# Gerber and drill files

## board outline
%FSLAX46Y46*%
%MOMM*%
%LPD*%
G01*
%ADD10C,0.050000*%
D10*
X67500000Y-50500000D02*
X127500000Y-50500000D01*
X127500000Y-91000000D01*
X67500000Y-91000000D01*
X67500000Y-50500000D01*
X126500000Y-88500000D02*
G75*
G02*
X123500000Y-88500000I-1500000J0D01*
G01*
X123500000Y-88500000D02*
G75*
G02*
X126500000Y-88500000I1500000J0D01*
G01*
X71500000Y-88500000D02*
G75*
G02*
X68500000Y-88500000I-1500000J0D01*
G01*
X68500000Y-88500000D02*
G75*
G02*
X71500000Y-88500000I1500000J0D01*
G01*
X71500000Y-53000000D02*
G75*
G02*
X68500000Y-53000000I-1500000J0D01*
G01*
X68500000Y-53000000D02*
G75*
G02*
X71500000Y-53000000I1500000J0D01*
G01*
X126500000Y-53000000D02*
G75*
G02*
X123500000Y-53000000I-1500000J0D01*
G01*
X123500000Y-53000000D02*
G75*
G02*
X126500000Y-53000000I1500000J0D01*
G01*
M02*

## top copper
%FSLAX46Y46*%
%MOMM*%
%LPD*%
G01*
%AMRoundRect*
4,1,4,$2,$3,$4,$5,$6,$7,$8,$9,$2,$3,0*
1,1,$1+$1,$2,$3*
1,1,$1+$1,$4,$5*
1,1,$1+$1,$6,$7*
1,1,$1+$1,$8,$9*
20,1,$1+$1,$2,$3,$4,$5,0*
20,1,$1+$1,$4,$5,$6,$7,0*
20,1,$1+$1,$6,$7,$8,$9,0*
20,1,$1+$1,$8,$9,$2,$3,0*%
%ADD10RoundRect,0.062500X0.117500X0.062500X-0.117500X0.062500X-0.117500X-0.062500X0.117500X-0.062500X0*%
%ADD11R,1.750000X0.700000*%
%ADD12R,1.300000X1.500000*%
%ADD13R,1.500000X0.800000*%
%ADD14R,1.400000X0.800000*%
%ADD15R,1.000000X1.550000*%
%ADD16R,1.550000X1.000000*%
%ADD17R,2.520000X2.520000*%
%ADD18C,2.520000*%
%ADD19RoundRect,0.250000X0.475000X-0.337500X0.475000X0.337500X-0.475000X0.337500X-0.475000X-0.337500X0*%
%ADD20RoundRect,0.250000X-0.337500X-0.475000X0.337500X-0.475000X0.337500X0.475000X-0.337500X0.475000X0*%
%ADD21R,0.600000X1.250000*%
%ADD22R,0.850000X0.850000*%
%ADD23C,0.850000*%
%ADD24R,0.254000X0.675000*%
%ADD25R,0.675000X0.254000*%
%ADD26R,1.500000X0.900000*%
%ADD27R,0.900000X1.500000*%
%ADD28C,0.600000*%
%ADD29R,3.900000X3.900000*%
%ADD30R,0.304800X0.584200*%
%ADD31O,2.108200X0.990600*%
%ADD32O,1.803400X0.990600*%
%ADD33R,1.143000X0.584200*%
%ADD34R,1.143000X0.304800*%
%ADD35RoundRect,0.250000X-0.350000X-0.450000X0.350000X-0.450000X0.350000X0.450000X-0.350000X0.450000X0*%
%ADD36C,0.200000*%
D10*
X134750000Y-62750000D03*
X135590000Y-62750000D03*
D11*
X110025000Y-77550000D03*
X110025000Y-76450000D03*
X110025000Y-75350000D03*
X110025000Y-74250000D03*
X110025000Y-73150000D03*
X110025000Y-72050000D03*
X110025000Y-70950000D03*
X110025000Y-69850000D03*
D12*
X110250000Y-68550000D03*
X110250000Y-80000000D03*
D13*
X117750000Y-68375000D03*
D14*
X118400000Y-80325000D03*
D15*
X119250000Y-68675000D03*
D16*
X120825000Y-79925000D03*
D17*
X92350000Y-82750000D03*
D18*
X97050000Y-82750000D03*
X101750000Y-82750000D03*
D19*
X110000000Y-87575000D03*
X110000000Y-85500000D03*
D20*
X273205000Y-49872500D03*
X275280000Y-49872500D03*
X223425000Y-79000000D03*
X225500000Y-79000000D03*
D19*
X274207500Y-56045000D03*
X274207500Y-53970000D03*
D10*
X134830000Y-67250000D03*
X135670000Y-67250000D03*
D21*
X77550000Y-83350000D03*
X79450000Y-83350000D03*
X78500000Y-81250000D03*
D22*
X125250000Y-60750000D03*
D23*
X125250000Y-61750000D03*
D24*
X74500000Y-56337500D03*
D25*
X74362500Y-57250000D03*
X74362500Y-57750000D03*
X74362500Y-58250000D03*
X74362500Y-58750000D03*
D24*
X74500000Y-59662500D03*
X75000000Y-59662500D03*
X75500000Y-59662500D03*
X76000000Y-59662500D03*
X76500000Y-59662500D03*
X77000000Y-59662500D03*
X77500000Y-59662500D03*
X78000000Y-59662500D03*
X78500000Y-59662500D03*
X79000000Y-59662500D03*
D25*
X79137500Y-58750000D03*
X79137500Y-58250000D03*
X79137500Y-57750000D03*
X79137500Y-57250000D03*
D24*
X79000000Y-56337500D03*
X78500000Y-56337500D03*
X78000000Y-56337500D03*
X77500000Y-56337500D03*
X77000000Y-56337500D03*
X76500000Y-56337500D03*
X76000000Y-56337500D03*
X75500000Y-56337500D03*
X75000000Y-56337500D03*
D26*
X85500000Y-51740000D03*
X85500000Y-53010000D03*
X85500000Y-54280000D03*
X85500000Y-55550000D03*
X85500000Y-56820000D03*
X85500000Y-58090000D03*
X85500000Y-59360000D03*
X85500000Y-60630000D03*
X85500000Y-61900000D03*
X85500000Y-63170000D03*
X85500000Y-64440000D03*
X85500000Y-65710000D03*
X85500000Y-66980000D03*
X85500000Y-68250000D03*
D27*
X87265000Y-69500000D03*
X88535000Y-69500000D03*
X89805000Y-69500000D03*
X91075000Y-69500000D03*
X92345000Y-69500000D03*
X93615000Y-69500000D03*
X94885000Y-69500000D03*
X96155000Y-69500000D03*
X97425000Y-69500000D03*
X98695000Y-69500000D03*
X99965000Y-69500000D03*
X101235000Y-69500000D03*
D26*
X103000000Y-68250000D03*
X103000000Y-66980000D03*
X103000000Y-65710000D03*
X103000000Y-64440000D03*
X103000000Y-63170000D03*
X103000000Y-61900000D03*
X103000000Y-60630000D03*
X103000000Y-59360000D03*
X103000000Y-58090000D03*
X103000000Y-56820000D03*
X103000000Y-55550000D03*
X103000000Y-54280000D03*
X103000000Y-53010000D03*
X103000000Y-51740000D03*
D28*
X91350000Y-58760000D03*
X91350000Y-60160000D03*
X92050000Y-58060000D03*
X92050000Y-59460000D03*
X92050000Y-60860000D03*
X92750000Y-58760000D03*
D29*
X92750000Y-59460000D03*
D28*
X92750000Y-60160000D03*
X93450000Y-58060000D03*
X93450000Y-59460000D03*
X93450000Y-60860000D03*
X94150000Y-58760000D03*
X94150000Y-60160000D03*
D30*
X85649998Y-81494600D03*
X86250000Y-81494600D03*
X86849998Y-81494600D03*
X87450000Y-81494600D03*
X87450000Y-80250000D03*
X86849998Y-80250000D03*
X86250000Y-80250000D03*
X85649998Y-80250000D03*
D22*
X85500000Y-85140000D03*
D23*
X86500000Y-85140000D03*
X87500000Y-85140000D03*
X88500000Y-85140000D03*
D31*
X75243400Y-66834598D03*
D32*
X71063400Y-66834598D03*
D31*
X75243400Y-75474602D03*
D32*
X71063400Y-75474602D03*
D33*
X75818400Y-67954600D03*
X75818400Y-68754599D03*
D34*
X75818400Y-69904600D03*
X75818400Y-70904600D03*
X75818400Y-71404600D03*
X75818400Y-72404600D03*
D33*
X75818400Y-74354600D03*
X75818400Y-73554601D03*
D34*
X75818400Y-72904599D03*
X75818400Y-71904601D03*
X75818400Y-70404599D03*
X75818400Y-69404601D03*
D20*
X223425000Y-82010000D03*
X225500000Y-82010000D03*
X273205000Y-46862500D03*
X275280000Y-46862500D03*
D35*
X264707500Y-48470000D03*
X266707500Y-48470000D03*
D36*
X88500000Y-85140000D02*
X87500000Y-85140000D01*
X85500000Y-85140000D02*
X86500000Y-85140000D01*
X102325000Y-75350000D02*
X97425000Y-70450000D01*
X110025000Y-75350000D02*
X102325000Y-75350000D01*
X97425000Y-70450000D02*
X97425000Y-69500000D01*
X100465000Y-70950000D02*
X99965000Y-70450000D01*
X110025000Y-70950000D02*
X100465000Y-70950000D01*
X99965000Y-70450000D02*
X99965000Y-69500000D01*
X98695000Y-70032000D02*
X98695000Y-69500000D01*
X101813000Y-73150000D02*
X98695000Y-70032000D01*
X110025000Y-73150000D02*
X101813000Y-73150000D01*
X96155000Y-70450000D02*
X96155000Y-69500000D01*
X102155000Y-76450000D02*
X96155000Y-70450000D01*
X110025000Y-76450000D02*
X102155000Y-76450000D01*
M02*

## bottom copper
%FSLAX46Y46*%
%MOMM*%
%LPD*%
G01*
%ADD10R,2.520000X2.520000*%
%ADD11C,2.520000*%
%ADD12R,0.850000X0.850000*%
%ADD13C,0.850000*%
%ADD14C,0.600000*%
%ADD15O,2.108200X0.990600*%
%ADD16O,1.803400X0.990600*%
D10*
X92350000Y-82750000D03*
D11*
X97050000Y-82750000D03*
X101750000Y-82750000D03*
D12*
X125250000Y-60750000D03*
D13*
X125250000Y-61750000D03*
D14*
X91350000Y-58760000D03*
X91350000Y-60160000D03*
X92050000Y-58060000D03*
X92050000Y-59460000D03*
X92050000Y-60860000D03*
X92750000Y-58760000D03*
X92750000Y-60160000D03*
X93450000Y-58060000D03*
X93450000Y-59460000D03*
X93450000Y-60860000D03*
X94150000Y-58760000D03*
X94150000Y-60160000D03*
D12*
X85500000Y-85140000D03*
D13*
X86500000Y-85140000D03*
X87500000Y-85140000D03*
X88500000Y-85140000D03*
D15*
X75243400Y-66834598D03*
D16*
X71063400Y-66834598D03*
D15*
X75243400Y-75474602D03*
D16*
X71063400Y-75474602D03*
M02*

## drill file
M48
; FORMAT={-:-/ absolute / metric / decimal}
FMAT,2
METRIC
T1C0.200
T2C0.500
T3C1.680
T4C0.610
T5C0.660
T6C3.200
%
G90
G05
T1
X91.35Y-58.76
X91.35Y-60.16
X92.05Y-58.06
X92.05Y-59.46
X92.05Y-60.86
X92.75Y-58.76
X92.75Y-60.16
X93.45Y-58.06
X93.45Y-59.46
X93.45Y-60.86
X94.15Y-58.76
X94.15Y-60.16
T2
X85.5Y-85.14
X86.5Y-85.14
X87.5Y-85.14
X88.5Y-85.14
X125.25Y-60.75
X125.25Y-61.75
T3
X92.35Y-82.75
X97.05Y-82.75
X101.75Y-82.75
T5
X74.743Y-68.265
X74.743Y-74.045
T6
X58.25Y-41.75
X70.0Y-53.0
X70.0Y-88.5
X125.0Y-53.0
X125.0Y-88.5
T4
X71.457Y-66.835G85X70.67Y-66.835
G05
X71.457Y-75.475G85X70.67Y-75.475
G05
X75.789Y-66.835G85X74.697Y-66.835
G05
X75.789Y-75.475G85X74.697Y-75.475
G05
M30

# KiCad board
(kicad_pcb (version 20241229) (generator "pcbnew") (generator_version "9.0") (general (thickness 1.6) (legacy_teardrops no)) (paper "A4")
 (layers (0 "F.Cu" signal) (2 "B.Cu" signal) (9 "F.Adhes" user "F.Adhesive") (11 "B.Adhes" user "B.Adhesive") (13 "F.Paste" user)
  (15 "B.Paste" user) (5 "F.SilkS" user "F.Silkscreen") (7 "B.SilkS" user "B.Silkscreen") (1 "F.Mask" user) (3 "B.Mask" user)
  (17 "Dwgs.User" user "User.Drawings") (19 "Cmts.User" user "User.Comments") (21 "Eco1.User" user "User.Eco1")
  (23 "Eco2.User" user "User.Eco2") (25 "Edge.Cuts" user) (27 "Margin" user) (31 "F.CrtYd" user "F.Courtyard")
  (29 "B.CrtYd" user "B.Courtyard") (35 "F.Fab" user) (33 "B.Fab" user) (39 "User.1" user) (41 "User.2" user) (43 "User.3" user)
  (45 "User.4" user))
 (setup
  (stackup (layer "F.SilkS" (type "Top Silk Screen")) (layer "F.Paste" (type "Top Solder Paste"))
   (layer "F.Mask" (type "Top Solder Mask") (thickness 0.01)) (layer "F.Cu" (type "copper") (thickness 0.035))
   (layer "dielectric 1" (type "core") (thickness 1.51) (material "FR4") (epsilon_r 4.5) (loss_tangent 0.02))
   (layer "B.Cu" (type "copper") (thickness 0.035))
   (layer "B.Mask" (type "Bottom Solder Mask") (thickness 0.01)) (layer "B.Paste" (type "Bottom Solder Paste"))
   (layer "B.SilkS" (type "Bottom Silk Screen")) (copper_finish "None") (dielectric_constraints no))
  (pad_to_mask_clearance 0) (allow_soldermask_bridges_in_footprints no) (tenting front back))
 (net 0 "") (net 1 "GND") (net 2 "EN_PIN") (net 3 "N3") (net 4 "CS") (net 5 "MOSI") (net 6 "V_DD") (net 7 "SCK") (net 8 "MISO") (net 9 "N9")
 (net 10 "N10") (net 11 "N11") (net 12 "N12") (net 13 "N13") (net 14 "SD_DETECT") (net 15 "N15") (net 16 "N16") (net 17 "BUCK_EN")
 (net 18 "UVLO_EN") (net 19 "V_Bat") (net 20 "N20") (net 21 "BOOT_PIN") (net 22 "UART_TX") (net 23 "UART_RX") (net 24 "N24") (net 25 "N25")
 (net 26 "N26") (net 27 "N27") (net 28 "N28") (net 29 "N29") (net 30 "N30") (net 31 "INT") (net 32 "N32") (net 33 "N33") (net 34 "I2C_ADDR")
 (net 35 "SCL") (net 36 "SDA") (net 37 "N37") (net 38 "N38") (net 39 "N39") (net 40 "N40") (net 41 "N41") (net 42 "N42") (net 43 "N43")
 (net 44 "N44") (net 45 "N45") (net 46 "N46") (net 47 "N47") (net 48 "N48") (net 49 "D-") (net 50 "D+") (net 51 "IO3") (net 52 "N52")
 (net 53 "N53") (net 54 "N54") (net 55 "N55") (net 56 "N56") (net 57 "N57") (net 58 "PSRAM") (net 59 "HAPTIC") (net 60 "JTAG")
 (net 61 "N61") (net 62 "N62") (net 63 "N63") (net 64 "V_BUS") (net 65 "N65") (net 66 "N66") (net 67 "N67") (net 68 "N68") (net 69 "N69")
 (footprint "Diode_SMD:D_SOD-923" (layer "F.Cu") (at 135.17 62.75)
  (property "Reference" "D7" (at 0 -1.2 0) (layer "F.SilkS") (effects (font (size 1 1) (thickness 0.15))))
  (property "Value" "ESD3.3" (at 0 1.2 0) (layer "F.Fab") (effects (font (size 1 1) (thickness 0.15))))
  (pad "1" smd roundrect (at -0.42 0 180) (size 0.36 0.25) (layers "F.Cu" "F.Mask" "F.Paste") (roundrect_rratio 0.25) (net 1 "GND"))
  (pad "2" smd roundrect (at 0.42 0 180) (size 0.36 0.25) (layers "F.Cu" "F.Mask" "F.Paste") (roundrect_rratio 0.25) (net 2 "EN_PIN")))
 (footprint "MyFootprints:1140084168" (layer "F.Cu") (at 115.375 74.275 -90)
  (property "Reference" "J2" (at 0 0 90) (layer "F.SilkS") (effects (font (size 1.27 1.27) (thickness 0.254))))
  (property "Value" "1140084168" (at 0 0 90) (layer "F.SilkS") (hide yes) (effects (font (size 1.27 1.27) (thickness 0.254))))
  (pad "1" smd rect (at 3.275 5.35 270) (size 0.7 1.75) (layers "F.Cu" "F.Mask" "F.Paste") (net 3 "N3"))
  (pad "2" smd rect (at 2.175 5.35 270) (size 0.7 1.75) (layers "F.Cu" "F.Mask" "F.Paste") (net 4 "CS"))
  (pad "3" smd rect (at 1.075 5.35 270) (size 0.7 1.75) (layers "F.Cu" "F.Mask" "F.Paste") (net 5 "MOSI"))
  (pad "4" smd rect (at -0.025 5.35 270) (size 0.7 1.75) (layers "F.Cu" "F.Mask" "F.Paste") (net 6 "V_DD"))
  (pad "5" smd rect (at -1.125 5.35 270) (size 0.7 1.75) (layers "F.Cu" "F.Mask" "F.Paste") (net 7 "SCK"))
  (pad "6" smd rect (at -2.225 5.35 270) (size 0.7 1.75) (layers "F.Cu" "F.Mask" "F.Paste") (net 1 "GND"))
  (pad "7" smd rect (at -3.325 5.35 270) (size 0.7 1.75) (layers "F.Cu" "F.Mask" "F.Paste") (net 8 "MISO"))
  (pad "8" smd rect (at -4.425 5.35 270) (size 0.7 1.75) (layers "F.Cu" "F.Mask" "F.Paste") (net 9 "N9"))
  (pad "9" smd rect (at -5.725 5.125) (size 1.3 1.5) (layers "F.Cu" "F.Mask" "F.Paste") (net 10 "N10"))
  (pad "10" smd rect (at 5.725 5.125) (size 1.3 1.5) (layers "F.Cu" "F.Mask" "F.Paste") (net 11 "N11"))
  (pad "11" smd rect (at -5.9 -2.375 270) (size 0.8 1.5) (layers "F.Cu" "F.Mask" "F.Paste") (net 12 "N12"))
  (pad "12" smd rect (at 6.05 -3.025 270) (size 0.8 1.4) (layers "F.Cu" "F.Mask" "F.Paste") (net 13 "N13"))
  (pad "CD1" smd rect (at -5.6 -3.875) (size 1 1.55) (layers "F.Cu" "F.Mask" "F.Paste") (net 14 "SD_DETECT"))
  (pad "CD2" smd rect (at 5.65 -5.45 270) (size 1 1.55) (layers "F.Cu" "F.Mask" "F.Paste") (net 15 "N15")))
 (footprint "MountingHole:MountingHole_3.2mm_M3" (layer "F.Cu") (at 58.25 41.75)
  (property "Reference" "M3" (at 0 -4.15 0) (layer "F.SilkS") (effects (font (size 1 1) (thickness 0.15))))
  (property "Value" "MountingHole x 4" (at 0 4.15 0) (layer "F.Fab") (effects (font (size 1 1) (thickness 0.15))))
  (pad "" np_thru_hole circle (at 0 0) (size 3.2 3.2) (drill 3.2) (layers "*.Cu" "*.Mask")))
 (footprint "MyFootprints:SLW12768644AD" (layer "F.Cu") (at 92.35 82.75)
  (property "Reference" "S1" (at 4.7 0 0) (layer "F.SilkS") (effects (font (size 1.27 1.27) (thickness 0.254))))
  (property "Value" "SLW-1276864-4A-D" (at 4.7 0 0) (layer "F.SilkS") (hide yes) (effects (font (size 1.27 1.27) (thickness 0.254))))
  (pad "1" thru_hole rect (at 0 0) (size 2.52 2.52) (drill 1.68) (layers "*.Cu" "*.Mask") (remove_unused_layers no) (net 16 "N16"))
  (pad "2" thru_hole circle (at 4.7 0) (size 2.52 2.52) (drill 1.68) (layers "*.Cu" "*.Mask") (remove_unused_layers no) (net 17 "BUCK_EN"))
  (pad "3" thru_hole circle (at 9.4 0) (size 2.52 2.52) (drill 1.68) (layers "*.Cu" "*.Mask") (remove_unused_layers no) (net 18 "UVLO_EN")))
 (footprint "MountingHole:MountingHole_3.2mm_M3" (layer "F.Cu") (at 70 88.5)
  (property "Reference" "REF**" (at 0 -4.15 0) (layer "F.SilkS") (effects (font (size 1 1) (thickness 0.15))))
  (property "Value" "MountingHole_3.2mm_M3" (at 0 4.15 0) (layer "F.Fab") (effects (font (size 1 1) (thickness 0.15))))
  (pad "" np_thru_hole circle (at 0 0) (size 3.2 3.2) (drill 3.2) (layers "*.Cu" "*.Mask")))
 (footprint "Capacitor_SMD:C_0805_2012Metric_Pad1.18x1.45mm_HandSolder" (layer "F.Cu") (at 110 86.5375 90)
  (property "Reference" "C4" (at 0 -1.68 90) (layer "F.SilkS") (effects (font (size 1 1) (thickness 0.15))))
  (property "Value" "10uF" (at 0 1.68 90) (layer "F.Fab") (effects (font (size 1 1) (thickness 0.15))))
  (pad "1" smd roundrect (at -1.0375 0 90) (size 1.175 1.45) (layers "F.Cu" "F.Mask" "F.Paste") (roundrect_rratio 0.212766) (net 6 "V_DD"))
  (pad "2" smd roundrect (at 1.0375 0 90) (size 1.175 1.45) (layers "F.Cu" "F.Mask" "F.Paste") (roundrect_rratio 0.212766) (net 1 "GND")))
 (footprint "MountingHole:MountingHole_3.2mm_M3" (layer "F.Cu") (at 125 88.5)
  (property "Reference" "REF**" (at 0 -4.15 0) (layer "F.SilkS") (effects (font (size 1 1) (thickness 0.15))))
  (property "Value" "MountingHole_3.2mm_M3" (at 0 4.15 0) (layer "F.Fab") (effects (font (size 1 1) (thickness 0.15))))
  (pad "" np_thru_hole circle (at 0 0) (size 3.2 3.2) (drill 3.2) (layers "*.Cu" "*.Mask")))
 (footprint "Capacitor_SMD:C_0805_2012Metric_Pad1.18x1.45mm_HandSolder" (layer "F.Cu") (at 274.2425 49.8725)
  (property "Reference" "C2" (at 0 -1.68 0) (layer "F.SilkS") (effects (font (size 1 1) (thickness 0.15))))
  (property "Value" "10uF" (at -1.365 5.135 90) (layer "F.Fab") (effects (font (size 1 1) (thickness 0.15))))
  (pad "1" smd roundrect (at -1.0375 0) (size 1.175 1.45) (layers "F.Cu" "F.Mask" "F.Paste") (roundrect_rratio 0.212766) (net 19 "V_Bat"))
  (pad "2" smd roundrect (at 1.0375 0) (size 1.175 1.45) (layers "F.Cu" "F.Mask" "F.Paste") (roundrect_rratio 0.212766) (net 1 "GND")))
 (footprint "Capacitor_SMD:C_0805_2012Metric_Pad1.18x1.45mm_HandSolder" (layer "F.Cu") (at 224.4625 79)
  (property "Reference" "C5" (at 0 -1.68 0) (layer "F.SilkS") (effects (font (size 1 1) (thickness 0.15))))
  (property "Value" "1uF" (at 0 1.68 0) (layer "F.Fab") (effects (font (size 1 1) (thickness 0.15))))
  (pad "1" smd roundrect (at -1.0375 0) (size 1.175 1.45) (layers "F.Cu" "F.Mask" "F.Paste") (roundrect_rratio 0.212766) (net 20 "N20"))
  (pad "2" smd roundrect (at 1.0375 0) (size 1.175 1.45) (layers "F.Cu" "F.Mask" "F.Paste") (roundrect_rratio 0.212766) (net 1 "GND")))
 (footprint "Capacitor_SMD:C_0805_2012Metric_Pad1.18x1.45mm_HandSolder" (layer "F.Cu") (at 274.2075 55.0075 90)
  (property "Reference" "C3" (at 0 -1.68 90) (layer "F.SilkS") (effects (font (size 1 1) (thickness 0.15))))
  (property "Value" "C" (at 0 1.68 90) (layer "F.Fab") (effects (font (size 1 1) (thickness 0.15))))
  (pad "1" smd roundrect (at -1.0375 0 90) (size 1.175 1.45) (layers "F.Cu" "F.Mask" "F.Paste") (roundrect_rratio 0.212766) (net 6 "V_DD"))
  (pad "2" smd roundrect (at 1.0375 0 90) (size 1.175 1.45) (layers "F.Cu" "F.Mask" "F.Paste") (roundrect_rratio 0.212766) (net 1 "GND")))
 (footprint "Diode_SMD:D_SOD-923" (layer "F.Cu") (at 135.25 67.25)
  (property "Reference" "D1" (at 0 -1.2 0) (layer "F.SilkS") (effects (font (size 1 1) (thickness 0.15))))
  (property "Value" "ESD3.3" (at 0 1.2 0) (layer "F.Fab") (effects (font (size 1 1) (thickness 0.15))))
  (pad "1" smd roundrect (at -0.42 0 180) (size 0.36 0.25) (layers "F.Cu" "F.Mask" "F.Paste") (roundrect_rratio 0.25) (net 1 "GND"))
  (pad "2" smd roundrect (at 0.42 0 180) (size 0.36 0.25) (layers "F.Cu" "F.Mask" "F.Paste") (roundrect_rratio 0.25) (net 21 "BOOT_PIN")))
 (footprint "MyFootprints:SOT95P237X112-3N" (layer "F.Cu") (at 78.5 82.3 90)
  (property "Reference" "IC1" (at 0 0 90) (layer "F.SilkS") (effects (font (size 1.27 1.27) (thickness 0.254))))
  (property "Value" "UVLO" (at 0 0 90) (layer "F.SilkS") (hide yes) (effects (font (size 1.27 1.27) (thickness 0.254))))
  (pad "1" smd rect (at -1.05 -0.95 180) (size 0.6 1.25) (layers "F.Cu" "F.Mask" "F.Paste") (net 18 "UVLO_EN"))
  (pad "2" smd rect (at -1.05 0.95 180) (size 0.6 1.25) (layers "F.Cu" "F.Mask" "F.Paste") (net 19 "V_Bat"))
  (pad "3" smd rect (at 1.05 0 180) (size 0.6 1.25) (layers "F.Cu" "F.Mask" "F.Paste") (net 1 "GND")))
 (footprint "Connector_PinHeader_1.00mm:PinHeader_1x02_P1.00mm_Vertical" (layer "F.Cu") (at 125.25 60.75)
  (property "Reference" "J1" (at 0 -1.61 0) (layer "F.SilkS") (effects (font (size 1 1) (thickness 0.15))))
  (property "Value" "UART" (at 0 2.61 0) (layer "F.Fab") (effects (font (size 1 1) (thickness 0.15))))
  (pad "1" thru_hole rect (at 0 0) (size 0.85 0.85) (drill 0.5) (layers "*.Cu" "*.Mask") (remove_unused_layers no) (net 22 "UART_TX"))
  (pad "2" thru_hole circle (at 0 1) (size 0.85 0.85) (drill 0.5) (layers "*.Cu" "*.Mask") (remove_unused_layers no) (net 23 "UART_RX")))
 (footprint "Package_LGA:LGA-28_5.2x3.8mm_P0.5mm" (layer "F.Cu") (at 76.75 58)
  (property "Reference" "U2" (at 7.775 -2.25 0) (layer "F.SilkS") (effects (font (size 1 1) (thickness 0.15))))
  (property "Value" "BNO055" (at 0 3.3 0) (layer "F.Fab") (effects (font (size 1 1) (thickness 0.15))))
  (pad "1" smd rect (at -2.25 -1.6625) (size 0.254 0.675) (layers "F.Cu" "F.Mask" "F.Paste") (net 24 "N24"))
  (pad "2" smd rect (at -2.3875 -0.75 90) (size 0.254 0.675) (layers "F.Cu" "F.Mask" "F.Paste") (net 1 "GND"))
  (pad "3" smd rect (at -2.3875 -0.25 90) (size 0.254 0.675) (layers "F.Cu" "F.Mask" "F.Paste") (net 6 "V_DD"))
  (pad "4" smd rect (at -2.3875 0.25 90) (size 0.254 0.675) (layers "F.Cu" "F.Mask" "F.Paste") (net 6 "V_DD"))
  (pad "5" smd rect (at -2.3875 0.75 90) (size 0.254 0.675) (layers "F.Cu" "F.Mask" "F.Paste") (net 1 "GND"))
  (pad "6" smd rect (at -2.25 1.6625) (size 0.254 0.675) (layers "F.Cu" "F.Mask" "F.Paste") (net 1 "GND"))
  (pad "7" smd rect (at -1.75 1.6625) (size 0.254 0.675) (layers "F.Cu" "F.Mask" "F.Paste") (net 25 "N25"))
  (pad "8" smd rect (at -1.25 1.6625) (size 0.254 0.675) (layers "F.Cu" "F.Mask" "F.Paste") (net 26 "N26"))
  (pad "9" smd rect (at -0.75 1.6625) (size 0.254 0.675) (layers "F.Cu" "F.Mask" "F.Paste") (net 20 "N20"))
  (pad "10" smd rect (at -0.25 1.6625) (size 0.254 0.675) (layers "F.Cu" "F.Mask" "F.Paste") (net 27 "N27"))
  (pad "11" smd rect (at 0.25 1.6625) (size 0.254 0.675) (layers "F.Cu" "F.Mask" "F.Paste") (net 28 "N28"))
  (pad "12" smd rect (at 0.75 1.6625) (size 0.254 0.675) (layers "F.Cu" "F.Mask" "F.Paste") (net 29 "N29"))
  (pad "13" smd rect (at 1.25 1.6625) (size 0.254 0.675) (layers "F.Cu" "F.Mask" "F.Paste") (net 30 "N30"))
  (pad "14" smd rect (at 1.75 1.6625) (size 0.254 0.675) (layers "F.Cu" "F.Mask" "F.Paste") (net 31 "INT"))
  (pad "15" smd rect (at 2.25 1.6625) (size 0.254 0.675) (layers "F.Cu" "F.Mask" "F.Paste") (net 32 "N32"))
  (pad "16" smd rect (at 2.3875 0.75 90) (size 0.254 0.675) (layers "F.Cu" "F.Mask" "F.Paste") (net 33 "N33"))
  (pad "17" smd rect (at 2.3875 0.25 90) (size 0.254 0.675) (layers "F.Cu" "F.Mask" "F.Paste") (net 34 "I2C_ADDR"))
  (pad "18" smd rect (at 2.3875 -0.25 90) (size 0.254 0.675) (layers "F.Cu" "F.Mask" "F.Paste") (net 1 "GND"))
  (pad "19" smd rect (at 2.3875 -0.75 90) (size 0.254 0.675) (layers "F.Cu" "F.Mask" "F.Paste") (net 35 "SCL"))
  (pad "20" smd rect (at 2.25 -1.6625) (size 0.254 0.675) (layers "F.Cu" "F.Mask" "F.Paste") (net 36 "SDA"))
  (pad "21" smd rect (at 1.75 -1.6625) (size 0.254 0.675) (layers "F.Cu" "F.Mask" "F.Paste") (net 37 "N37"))
  (pad "22" smd rect (at 1.25 -1.6625) (size 0.254 0.675) (layers "F.Cu" "F.Mask" "F.Paste") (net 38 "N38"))
  (pad "23" smd rect (at 0.75 -1.6625) (size 0.254 0.675) (layers "F.Cu" "F.Mask" "F.Paste") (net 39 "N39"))
  (pad "24" smd rect (at 0.25 -1.6625) (size 0.254 0.675) (layers "F.Cu" "F.Mask" "F.Paste") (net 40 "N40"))
  (pad "25" smd rect (at -0.25 -1.6625) (size 0.254 0.675) (layers "F.Cu" "F.Mask" "F.Paste") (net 1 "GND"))
  (pad "26" smd rect (at -0.75 -1.6625) (size 0.254 0.675) (layers "F.Cu" "F.Mask" "F.Paste") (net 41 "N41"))
  (pad "27" smd rect (at -1.25 -1.6625) (size 0.254 0.675) (layers "F.Cu" "F.Mask" "F.Paste") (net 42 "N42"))
  (pad "28" smd rect (at -1.75 -1.6625) (size 0.254 0.675) (layers "F.Cu" "F.Mask" "F.Paste") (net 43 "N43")))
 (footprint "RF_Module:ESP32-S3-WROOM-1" (layer "F.Cu") (at 94.25 57)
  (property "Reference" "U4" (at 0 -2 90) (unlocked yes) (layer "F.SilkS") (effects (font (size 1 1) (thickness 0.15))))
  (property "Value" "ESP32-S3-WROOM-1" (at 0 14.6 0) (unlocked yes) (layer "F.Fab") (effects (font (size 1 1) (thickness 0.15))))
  (pad "" smd rect (at -2.9 1.06) (size 0.9 0.9) (layers "F.Paste"))
  (pad "" smd rect (at -2.9 2.46 270) (size 0.9 0.9) (layers "F.Paste"))
  (pad "" smd rect (at -2.9 3.86) (size 0.9 0.9) (layers "F.Paste"))
  (pad "" smd rect (at -1.5 1.06 270) (size 0.9 0.9) (layers "F.Paste"))
  (pad "" smd rect (at -1.5 2.46 270) (size 0.9 0.9) (layers "F.Paste"))
  (pad "" smd rect (at -1.5 3.86 270) (size 0.9 0.9) (layers "F.Paste"))
  (pad "" smd rect (at -0.1 1.06 270) (size 0.9 0.9) (layers "F.Paste"))
  (pad "" smd rect (at -0.1 2.46 270) (size 0.9 0.9) (layers "F.Paste"))
  (pad "" smd rect (at -0.1 3.86 270) (size 0.9 0.9) (layers "F.Paste"))
  (pad "1" smd rect (at -8.75 -5.26) (size 1.5 0.9) (layers "F.Cu" "F.Mask" "F.Paste") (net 1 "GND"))
  (pad "2" smd rect (at -8.75 -3.99) (size 1.5 0.9) (layers "F.Cu" "F.Mask" "F.Paste") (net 6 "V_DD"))
  (pad "3" smd rect (at -8.75 -2.72) (size 1.5 0.9) (layers "F.Cu" "F.Mask" "F.Paste") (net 2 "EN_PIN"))
  (pad "4" smd rect (at -8.75 -1.45) (size 1.5 0.9) (layers "F.Cu" "F.Mask" "F.Paste") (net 36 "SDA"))
  (pad "5" smd rect (at -8.75 -0.18) (size 1.5 0.9) (layers "F.Cu" "F.Mask" "F.Paste") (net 35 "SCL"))
  (pad "6" smd rect (at -8.75 1.09) (size 1.5 0.9) (layers "F.Cu" "F.Mask" "F.Paste") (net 34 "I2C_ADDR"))
  (pad "7" smd rect (at -8.75 2.36) (size 1.5 0.9) (layers "F.Cu" "F.Mask" "F.Paste") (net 31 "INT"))
  (pad "8" smd rect (at -8.75 3.63) (size 1.5 0.9) (layers "F.Cu" "F.Mask" "F.Paste") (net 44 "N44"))
  (pad "9" smd rect (at -8.75 4.9) (size 1.5 0.9) (layers "F.Cu" "F.Mask" "F.Paste") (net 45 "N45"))
  (pad "10" smd rect (at -8.75 6.17) (size 1.5 0.9) (layers "F.Cu" "F.Mask" "F.Paste") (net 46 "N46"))
  (pad "11" smd rect (at -8.75 7.44) (size 1.5 0.9) (layers "F.Cu" "F.Mask" "F.Paste") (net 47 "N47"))
  (pad "12" smd rect (at -8.75 8.71) (size 1.5 0.9) (layers "F.Cu" "F.Mask" "F.Paste") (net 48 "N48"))
  (pad "13" smd rect (at -8.75 9.98) (size 1.5 0.9) (layers "F.Cu" "F.Mask" "F.Paste") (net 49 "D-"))
  (pad "14" smd rect (at -8.75 11.25 180) (size 1.5 0.9) (layers "F.Cu" "F.Mask" "F.Paste") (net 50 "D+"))
  (pad "15" smd rect (at -6.985 12.5 270) (size 1.5 0.9) (layers "F.Cu" "F.Mask" "F.Paste") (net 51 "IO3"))
  (pad "16" smd rect (at -5.715 12.5 270) (size 1.5 0.9) (layers "F.Cu" "F.Mask" "F.Paste") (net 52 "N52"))
  (pad "17" smd rect (at -4.445 12.5 270) (size 1.5 0.9) (layers "F.Cu" "F.Mask" "F.Paste") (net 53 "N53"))
  (pad "18" smd rect (at -3.175 12.5 270) (size 1.5 0.9) (layers "F.Cu" "F.Mask" "F.Paste") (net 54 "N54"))
  (pad "19" smd rect (at -1.905 12.5 270) (size 1.5 0.9) (layers "F.Cu" "F.Mask" "F.Paste") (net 14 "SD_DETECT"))
  (pad "20" smd rect (at -0.635 12.5 270) (size 1.5 0.9) (layers "F.Cu" "F.Mask" "F.Paste") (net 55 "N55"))
  (pad "21" smd rect (at 0.635 12.5 270) (size 1.5 0.9) (layers "F.Cu" "F.Mask" "F.Paste") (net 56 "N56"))
  (pad "22" smd rect (at 1.905 12.5 270) (size 1.5 0.9) (layers "F.Cu" "F.Mask" "F.Paste") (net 4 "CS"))
  (pad "23" smd rect (at 3.175 12.5 270) (size 1.5 0.9) (layers "F.Cu" "F.Mask" "F.Paste") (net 5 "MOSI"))
  (pad "24" smd rect (at 4.445 12.5 270) (size 1.5 0.9) (layers "F.Cu" "F.Mask" "F.Paste") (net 7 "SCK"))
  (pad "25" smd rect (at 5.715 12.5 270) (size 1.5 0.9) (layers "F.Cu" "F.Mask" "F.Paste") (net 8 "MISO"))
  (pad "26" smd rect (at 6.985 12.5 270) (size 1.5 0.9) (layers "F.Cu" "F.Mask" "F.Paste") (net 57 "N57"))
  (pad "27" smd rect (at 8.75 11.25) (size 1.5 0.9) (layers "F.Cu" "F.Mask" "F.Paste") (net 21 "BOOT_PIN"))
  (pad "28" smd rect (at 8.75 9.98) (size 1.5 0.9) (layers "F.Cu" "F.Mask" "F.Paste") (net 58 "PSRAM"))
  (pad "29" smd rect (at 8.75 8.71) (size 1.5 0.9) (layers "F.Cu" "F.Mask" "F.Paste") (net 58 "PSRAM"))
  (pad "30" smd rect (at 8.75 7.44) (size 1.5 0.9) (layers "F.Cu" "F.Mask" "F.Paste") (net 58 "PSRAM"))
  (pad "31" smd rect (at 8.75 6.17) (size 1.5 0.9) (layers "F.Cu" "F.Mask" "F.Paste") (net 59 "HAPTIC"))
  (pad "32" smd rect (at 8.75 4.9) (size 1.5 0.9) (layers "F.Cu" "F.Mask" "F.Paste") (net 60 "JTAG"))
  (pad "33" smd rect (at 8.75 3.63) (size 1.5 0.9) (layers "F.Cu" "F.Mask" "F.Paste") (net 60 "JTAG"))
  (pad "34" smd rect (at 8.75 2.36) (size 1.5 0.9) (layers "F.Cu" "F.Mask" "F.Paste") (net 60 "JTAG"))
  (pad "35" smd rect (at 8.75 1.09) (size 1.5 0.9) (layers "F.Cu" "F.Mask" "F.Paste") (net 60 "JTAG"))
  (pad "36" smd rect (at 8.75 -0.18) (size 1.5 0.9) (layers "F.Cu" "F.Mask" "F.Paste") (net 23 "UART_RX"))
  (pad "37" smd rect (at 8.75 -1.45) (size 1.5 0.9) (layers "F.Cu" "F.Mask" "F.Paste") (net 22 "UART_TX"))
  (pad "38" smd rect (at 8.75 -2.72) (size 1.5 0.9) (layers "F.Cu" "F.Mask" "F.Paste") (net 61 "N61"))
  (pad "39" smd rect (at 8.75 -3.99) (size 1.5 0.9) (layers "F.Cu" "F.Mask" "F.Paste") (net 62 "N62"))
  (pad "40" smd rect (at 8.75 -5.26) (size 1.5 0.9) (layers "F.Cu" "F.Mask" "F.Paste") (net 1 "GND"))
  (pad "41" thru_hole circle (at -2.9 1.76 90) (size 0.6 0.6) (drill 0.2) (layers "*.Cu" "F.Mask") (remove_unused_layers no) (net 1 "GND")
   (zone_connect 2))
  (pad "41" thru_hole circle (at -2.9 3.16) (size 0.6 0.6) (drill 0.2) (layers "*.Cu" "F.Mask") (remove_unused_layers no) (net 1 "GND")
   (zone_connect 2))
  (pad "41" thru_hole circle (at -2.2 1.06) (size 0.6 0.6) (drill 0.2) (layers "*.Cu" "F.Mask") (remove_unused_layers no) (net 1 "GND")
   (zone_connect 2))
  (pad "41" thru_hole circle (at -2.2 2.46) (size 0.6 0.6) (drill 0.2) (layers "*.Cu" "F.Mask") (remove_unused_layers no) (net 1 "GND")
   (zone_connect 2))
  (pad "41" thru_hole circle (at -2.2 3.86) (size 0.6 0.6) (drill 0.2) (layers "*.Cu" "F.Mask") (remove_unused_layers no) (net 1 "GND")
   (zone_connect 2))
  (pad "41" thru_hole circle (at -1.5 1.76) (size 0.6 0.6) (drill 0.2) (layers "*.Cu" "F.Mask") (remove_unused_layers no) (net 1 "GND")
   (zone_connect 2))
  (pad "41" smd rect (at -1.5 2.46 270) (size 3.9 3.9) (layers "F.Cu" "F.Mask") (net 1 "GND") (zone_connect 2))
  (pad "41" thru_hole circle (at -1.5 3.16) (size 0.6 0.6) (drill 0.2) (layers "*.Cu" "F.Mask") (remove_unused_layers no) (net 1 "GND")
   (zone_connect 2))
  (pad "41" thru_hole circle (at -0.8 1.06) (size 0.6 0.6) (drill 0.2) (layers "*.Cu" "F.Mask") (remove_unused_layers no) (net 1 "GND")
   (zone_connect 2))
  (pad "41" thru_hole circle (at -0.8 2.46) (size 0.6 0.6) (drill 0.2) (layers "*.Cu" "F.Mask") (remove_unused_layers no) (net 1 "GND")
   (zone_connect 2))
  (pad "41" thru_hole circle (at -0.8 3.86) (size 0.6 0.6) (drill 0.2) (layers "*.Cu" "F.Mask") (remove_unused_layers no) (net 1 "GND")
   (zone_connect 2))
  (pad "41" thru_hole circle (at -0.1 1.76) (size 0.6 0.6) (drill 0.2) (layers "*.Cu" "F.Mask") (remove_unused_layers no) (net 1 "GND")
   (zone_connect 2))
  (pad "41" thru_hole circle (at -0.1 3.16) (size 0.6 0.6) (drill 0.2) (layers "*.Cu" "F.Mask") (remove_unused_layers no) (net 1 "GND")
   (zone_connect 2))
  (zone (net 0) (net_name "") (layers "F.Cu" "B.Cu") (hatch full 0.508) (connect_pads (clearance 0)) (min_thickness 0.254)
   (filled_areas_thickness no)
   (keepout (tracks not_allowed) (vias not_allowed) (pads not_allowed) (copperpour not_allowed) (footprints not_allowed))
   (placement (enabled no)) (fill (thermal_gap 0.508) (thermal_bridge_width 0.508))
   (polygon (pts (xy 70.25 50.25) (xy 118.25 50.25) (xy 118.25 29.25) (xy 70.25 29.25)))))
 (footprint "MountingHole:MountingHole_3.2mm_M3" (layer "F.Cu") (at 70 53)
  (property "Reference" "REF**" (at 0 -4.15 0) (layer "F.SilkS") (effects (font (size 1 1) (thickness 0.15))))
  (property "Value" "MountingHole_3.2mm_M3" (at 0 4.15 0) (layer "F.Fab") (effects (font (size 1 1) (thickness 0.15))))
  (pad "" np_thru_hole circle (at 0 0) (size 3.2 3.2) (drill 3.2) (layers "*.Cu" "*.Mask")))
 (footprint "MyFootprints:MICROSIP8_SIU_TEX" (layer "F.Cu") (at 86.549999 80.8723 90)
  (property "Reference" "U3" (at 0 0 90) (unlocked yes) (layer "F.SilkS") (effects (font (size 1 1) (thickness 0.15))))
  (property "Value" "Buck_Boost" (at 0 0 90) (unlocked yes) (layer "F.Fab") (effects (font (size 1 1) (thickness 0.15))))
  (pad "1" smd rect (at -0.6223 -0.900001 90) (size 0.5842 0.3048) (layers "F.Cu" "F.Mask" "F.Paste") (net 19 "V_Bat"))
  (pad "2" smd rect (at -0.6223 -0.299999 90) (size 0.5842 0.3048) (layers "F.Cu" "F.Mask" "F.Paste") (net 1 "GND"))
  (pad "3" smd rect (at -0.6223 0.299999 90) (size 0.5842 0.3048) (layers "F.Cu" "F.Mask" "F.Paste") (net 1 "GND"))
  (pad "4" smd rect (at -0.6223 0.900001 90) (size 0.5842 0.3048) (layers "F.Cu" "F.Mask" "F.Paste") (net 6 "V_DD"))
  (pad "5" smd rect (at 0.6223 0.900001 90) (size 0.5842 0.3048) (layers "F.Cu" "F.Mask" "F.Paste") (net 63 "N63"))
  (pad "6" smd rect (at 0.6223 0.299999 90) (size 0.5842 0.3048) (layers "F.Cu" "F.Mask" "F.Paste") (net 1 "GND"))
  (pad "7" smd rect (at 0.6223 -0.299999 90) (size 0.5842 0.3048) (layers "F.Cu" "F.Mask" "F.Paste") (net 6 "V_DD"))
  (pad "8" smd rect (at 0.6223 -0.900001 90) (size 0.5842 0.3048) (layers "F.Cu" "F.Mask" "F.Paste") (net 17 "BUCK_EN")))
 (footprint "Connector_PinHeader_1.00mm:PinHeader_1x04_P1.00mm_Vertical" (layer "F.Cu") (at 85.5 85.14 90)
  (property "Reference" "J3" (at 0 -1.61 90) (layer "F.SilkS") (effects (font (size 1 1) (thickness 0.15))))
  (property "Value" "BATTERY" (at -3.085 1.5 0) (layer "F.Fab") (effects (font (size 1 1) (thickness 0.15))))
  (pad "1" thru_hole rect (at 0 0 90) (size 0.85 0.85) (drill 0.5) (layers "*.Cu" "*.Mask") (remove_unused_layers no) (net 19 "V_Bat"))
  (pad "2" thru_hole circle (at 0 1 90) (size 0.85 0.85) (drill 0.5) (layers "*.Cu" "*.Mask") (remove_unused_layers no) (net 19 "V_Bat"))
  (pad "3" thru_hole circle (at 0 2 90) (size 0.85 0.85) (drill 0.5) (layers "*.Cu" "*.Mask") (remove_unused_layers no) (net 1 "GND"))
  (pad "4" thru_hole circle (at 0 3 90) (size 0.85 0.85) (drill 0.5) (layers "*.Cu" "*.Mask") (remove_unused_layers no) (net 1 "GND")))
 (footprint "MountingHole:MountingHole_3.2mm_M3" (layer "F.Cu") (at 125 53)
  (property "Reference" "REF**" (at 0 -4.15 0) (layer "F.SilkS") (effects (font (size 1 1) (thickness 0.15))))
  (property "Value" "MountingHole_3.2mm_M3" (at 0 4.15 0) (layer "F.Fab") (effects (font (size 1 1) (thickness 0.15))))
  (pad "" np_thru_hole circle (at 0 0) (size 3.2 3.2) (drill 3.2) (layers "*.Cu" "*.Mask")))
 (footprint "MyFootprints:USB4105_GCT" (layer "F.Cu") (at 72.3326 71.1546 -90)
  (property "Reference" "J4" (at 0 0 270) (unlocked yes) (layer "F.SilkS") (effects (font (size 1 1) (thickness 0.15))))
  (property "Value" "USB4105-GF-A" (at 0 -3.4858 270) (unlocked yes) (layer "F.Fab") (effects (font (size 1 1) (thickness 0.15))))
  (pad "" np_thru_hole oval (at -4.320002 -2.9108 270) (size 0.9906 2.1082) (drill oval 0.6096 1.7018) (layers "*.Cu" "*.Mask"))
  (pad "" np_thru_hole oval (at -4.320002 1.2692 270) (size 0.9906 1.8034) (drill oval 0.6096 1.397) (layers "*.Cu" "*.Mask"))
  (pad "" np_thru_hole circle (at -2.889999 -2.410801 270) (size 0.6604 0.6604) (drill 0.6604) (layers "*.Cu" "*.Mask"))
  (pad "" np_thru_hole circle (at 2.889999 -2.410801 270) (size 0.6604 0.6604) (drill 0.6604) (layers "*.Cu" "*.Mask"))
  (pad "" np_thru_hole oval (at 4.320002 -2.9108 270) (size 0.9906 2.1082) (drill oval 0.6096 1.7018) (layers "*.Cu" "*.Mask"))
  (pad "" np_thru_hole oval (at 4.320002 1.2692 270) (size 0.9906 1.8034) (drill oval 0.6096 1.397) (layers "*.Cu" "*.Mask"))
  (pad "A1-B12" smd rect (at -3.2 -3.4858 270) (size 0.5842 1.143) (layers "F.Cu" "F.Mask" "F.Paste") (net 1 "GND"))
  (pad "A4-B9" smd rect (at -2.400001 -3.4858 270) (size 0.5842 1.143) (layers "F.Cu" "F.Mask" "F.Paste") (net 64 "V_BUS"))
  (pad "A5" smd rect (at -1.25 -3.4858 270) (size 0.3048 1.143) (layers "F.Cu" "F.Mask" "F.Paste") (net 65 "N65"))
  (pad "A6" smd rect (at -0.25 -3.4858 270) (size 0.3048 1.143) (layers "F.Cu" "F.Mask" "F.Paste") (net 50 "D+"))
  (pad "A7" smd rect (at 0.25 -3.4858 270) (size 0.3048 1.143) (layers "F.Cu" "F.Mask" "F.Paste") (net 49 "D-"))
  (pad "A8" smd rect (at 1.25 -3.4858 270) (size 0.3048 1.143) (layers "F.Cu" "F.Mask" "F.Paste") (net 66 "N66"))
  (pad "B1-A12" smd rect (at 3.2 -3.4858 270) (size 0.5842 1.143) (layers "F.Cu" "F.Mask" "F.Paste") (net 1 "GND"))
  (pad "B4-A9" smd rect (at 2.400001 -3.4858 270) (size 0.5842 1.143) (layers "F.Cu" "F.Mask" "F.Paste") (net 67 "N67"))
  (pad "B5" smd rect (at 1.749999 -3.4858 270) (size 0.3048 1.143) (layers "F.Cu" "F.Mask" "F.Paste") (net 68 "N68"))
  (pad "B6" smd rect (at 0.750001 -3.4858 270) (size 0.3048 1.143) (layers "F.Cu" "F.Mask" "F.Paste") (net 50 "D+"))
  (pad "B7" smd rect (at -0.750001 -3.4858 270) (size 0.3048 1.143) (layers "F.Cu" "F.Mask" "F.Paste") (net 49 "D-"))
  (pad "B8" smd rect (at -1.749999 -3.4858 270) (size 0.3048 1.143) (layers "F.Cu" "F.Mask" "F.Paste") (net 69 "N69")))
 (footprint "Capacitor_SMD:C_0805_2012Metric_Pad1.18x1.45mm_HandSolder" (layer "F.Cu") (at 224.4625 82.01)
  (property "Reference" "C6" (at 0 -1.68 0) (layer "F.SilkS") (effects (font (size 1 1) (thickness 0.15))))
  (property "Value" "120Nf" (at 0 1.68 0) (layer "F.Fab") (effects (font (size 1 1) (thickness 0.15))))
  (pad "1" smd roundrect (at -1.0375 0) (size 1.175 1.45) (layers "F.Cu" "F.Mask" "F.Paste") (roundrect_rratio 0.212766) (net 1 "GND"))
  (pad "2" smd roundrect (at 1.0375 0) (size 1.175 1.45) (layers "F.Cu" "F.Mask" "F.Paste") (roundrect_rratio 0.212766) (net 43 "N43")))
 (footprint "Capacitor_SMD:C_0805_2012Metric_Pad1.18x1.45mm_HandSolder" (layer "F.Cu") (at 274.2425 46.8625)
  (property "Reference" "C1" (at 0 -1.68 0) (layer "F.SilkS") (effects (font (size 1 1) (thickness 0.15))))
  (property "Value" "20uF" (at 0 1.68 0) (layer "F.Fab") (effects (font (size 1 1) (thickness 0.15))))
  (pad "1" smd roundrect (at -1.0375 0) (size 1.175 1.45) (layers "F.Cu" "F.Mask" "F.Paste") (roundrect_rratio 0.212766) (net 1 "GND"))
  (pad "2" smd roundrect (at 1.0375 0) (size 1.175 1.45) (layers "F.Cu" "F.Mask" "F.Paste") (roundrect_rratio 0.212766) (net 6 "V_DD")))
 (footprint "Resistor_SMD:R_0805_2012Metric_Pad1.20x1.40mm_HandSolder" (layer "F.Cu") (at 265.7075 48.47)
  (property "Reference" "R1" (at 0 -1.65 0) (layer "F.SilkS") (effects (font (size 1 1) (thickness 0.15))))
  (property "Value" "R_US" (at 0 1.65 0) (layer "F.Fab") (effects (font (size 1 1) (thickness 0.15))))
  (pad "1" smd roundrect (at -1 0) (size 1.2 1.4) (layers "F.Cu" "F.Mask" "F.Paste") (roundrect_rratio 0.208333) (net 19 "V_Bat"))
  (pad "2" smd roundrect (at 1 0) (size 1.2 1.4) (layers "F.Cu" "F.Mask" "F.Paste") (roundrect_rratio 0.208333) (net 18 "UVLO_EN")))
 (gr_rect (start 67.5 50.5) (end 127.5 91) (stroke (width 0.05) (type solid)) (fill no) (layer "Edge.Cuts"))
 (gr_circle (center 125 88.5) (end 126.5 88.5) (stroke (width 0.05) (type solid)) (fill no) (layer "Edge.Cuts"))
 (gr_circle (center 70 88.5) (end 71.5 88.5) (stroke (width 0.05) (type solid)) (fill no) (layer "Edge.Cuts"))
 (gr_circle (center 70 53) (end 71.5 53) (stroke (width 0.05) (type solid)) (fill no) (layer "Edge.Cuts"))
 (gr_circle (center 125 53) (end 126.5 53) (stroke (width 0.05) (type solid)) (fill no) (layer "Edge.Cuts"))
 (segment (start 88.5 85.14) (end 87.5 85.14) (width 0.2) (layer "F.Cu") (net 1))
 (segment (start 85.5 85.14) (end 86.5 85.14) (width 0.2) (layer "F.Cu") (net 19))
 (segment (start 102.325 75.35) (end 97.425 70.45) (width 0.2) (layer "F.Cu") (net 5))
 (segment (start 110.025 75.35) (end 102.325 75.35) (width 0.2) (layer "F.Cu") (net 5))
 (segment (start 97.425 70.45) (end 97.425 69.5) (width 0.2) (layer "F.Cu") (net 5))
 (segment (start 100.465 70.95) (end 99.965 70.45) (width 0.2) (layer "F.Cu") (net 8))
 (segment (start 110.025 70.95) (end 100.465 70.95) (width 0.2) (layer "F.Cu") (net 8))
 (segment (start 99.965 70.45) (end 99.965 69.5) (width 0.2) (layer "F.Cu") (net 8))
 (segment (start 98.695 70.032) (end 98.695 69.5) (width 0.2) (layer "F.Cu") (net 7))
 (segment (start 101.813 73.15) (end 98.695 70.032) (width 0.2) (layer "F.Cu") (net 7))
 (segment (start 110.025 73.15) (end 101.813 73.15) (width 0.2) (layer "F.Cu") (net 7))
 (segment (start 96.155 70.45) (end 96.155 69.5) (width 0.2) (layer "F.Cu") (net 4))
 (segment (start 102.155 76.45) (end 96.155 70.45) (width 0.2) (layer "F.Cu") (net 4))
 (segment (start 110.025 76.45) (end 102.155 76.45) (width 0.2) (layer "F.Cu") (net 4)))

